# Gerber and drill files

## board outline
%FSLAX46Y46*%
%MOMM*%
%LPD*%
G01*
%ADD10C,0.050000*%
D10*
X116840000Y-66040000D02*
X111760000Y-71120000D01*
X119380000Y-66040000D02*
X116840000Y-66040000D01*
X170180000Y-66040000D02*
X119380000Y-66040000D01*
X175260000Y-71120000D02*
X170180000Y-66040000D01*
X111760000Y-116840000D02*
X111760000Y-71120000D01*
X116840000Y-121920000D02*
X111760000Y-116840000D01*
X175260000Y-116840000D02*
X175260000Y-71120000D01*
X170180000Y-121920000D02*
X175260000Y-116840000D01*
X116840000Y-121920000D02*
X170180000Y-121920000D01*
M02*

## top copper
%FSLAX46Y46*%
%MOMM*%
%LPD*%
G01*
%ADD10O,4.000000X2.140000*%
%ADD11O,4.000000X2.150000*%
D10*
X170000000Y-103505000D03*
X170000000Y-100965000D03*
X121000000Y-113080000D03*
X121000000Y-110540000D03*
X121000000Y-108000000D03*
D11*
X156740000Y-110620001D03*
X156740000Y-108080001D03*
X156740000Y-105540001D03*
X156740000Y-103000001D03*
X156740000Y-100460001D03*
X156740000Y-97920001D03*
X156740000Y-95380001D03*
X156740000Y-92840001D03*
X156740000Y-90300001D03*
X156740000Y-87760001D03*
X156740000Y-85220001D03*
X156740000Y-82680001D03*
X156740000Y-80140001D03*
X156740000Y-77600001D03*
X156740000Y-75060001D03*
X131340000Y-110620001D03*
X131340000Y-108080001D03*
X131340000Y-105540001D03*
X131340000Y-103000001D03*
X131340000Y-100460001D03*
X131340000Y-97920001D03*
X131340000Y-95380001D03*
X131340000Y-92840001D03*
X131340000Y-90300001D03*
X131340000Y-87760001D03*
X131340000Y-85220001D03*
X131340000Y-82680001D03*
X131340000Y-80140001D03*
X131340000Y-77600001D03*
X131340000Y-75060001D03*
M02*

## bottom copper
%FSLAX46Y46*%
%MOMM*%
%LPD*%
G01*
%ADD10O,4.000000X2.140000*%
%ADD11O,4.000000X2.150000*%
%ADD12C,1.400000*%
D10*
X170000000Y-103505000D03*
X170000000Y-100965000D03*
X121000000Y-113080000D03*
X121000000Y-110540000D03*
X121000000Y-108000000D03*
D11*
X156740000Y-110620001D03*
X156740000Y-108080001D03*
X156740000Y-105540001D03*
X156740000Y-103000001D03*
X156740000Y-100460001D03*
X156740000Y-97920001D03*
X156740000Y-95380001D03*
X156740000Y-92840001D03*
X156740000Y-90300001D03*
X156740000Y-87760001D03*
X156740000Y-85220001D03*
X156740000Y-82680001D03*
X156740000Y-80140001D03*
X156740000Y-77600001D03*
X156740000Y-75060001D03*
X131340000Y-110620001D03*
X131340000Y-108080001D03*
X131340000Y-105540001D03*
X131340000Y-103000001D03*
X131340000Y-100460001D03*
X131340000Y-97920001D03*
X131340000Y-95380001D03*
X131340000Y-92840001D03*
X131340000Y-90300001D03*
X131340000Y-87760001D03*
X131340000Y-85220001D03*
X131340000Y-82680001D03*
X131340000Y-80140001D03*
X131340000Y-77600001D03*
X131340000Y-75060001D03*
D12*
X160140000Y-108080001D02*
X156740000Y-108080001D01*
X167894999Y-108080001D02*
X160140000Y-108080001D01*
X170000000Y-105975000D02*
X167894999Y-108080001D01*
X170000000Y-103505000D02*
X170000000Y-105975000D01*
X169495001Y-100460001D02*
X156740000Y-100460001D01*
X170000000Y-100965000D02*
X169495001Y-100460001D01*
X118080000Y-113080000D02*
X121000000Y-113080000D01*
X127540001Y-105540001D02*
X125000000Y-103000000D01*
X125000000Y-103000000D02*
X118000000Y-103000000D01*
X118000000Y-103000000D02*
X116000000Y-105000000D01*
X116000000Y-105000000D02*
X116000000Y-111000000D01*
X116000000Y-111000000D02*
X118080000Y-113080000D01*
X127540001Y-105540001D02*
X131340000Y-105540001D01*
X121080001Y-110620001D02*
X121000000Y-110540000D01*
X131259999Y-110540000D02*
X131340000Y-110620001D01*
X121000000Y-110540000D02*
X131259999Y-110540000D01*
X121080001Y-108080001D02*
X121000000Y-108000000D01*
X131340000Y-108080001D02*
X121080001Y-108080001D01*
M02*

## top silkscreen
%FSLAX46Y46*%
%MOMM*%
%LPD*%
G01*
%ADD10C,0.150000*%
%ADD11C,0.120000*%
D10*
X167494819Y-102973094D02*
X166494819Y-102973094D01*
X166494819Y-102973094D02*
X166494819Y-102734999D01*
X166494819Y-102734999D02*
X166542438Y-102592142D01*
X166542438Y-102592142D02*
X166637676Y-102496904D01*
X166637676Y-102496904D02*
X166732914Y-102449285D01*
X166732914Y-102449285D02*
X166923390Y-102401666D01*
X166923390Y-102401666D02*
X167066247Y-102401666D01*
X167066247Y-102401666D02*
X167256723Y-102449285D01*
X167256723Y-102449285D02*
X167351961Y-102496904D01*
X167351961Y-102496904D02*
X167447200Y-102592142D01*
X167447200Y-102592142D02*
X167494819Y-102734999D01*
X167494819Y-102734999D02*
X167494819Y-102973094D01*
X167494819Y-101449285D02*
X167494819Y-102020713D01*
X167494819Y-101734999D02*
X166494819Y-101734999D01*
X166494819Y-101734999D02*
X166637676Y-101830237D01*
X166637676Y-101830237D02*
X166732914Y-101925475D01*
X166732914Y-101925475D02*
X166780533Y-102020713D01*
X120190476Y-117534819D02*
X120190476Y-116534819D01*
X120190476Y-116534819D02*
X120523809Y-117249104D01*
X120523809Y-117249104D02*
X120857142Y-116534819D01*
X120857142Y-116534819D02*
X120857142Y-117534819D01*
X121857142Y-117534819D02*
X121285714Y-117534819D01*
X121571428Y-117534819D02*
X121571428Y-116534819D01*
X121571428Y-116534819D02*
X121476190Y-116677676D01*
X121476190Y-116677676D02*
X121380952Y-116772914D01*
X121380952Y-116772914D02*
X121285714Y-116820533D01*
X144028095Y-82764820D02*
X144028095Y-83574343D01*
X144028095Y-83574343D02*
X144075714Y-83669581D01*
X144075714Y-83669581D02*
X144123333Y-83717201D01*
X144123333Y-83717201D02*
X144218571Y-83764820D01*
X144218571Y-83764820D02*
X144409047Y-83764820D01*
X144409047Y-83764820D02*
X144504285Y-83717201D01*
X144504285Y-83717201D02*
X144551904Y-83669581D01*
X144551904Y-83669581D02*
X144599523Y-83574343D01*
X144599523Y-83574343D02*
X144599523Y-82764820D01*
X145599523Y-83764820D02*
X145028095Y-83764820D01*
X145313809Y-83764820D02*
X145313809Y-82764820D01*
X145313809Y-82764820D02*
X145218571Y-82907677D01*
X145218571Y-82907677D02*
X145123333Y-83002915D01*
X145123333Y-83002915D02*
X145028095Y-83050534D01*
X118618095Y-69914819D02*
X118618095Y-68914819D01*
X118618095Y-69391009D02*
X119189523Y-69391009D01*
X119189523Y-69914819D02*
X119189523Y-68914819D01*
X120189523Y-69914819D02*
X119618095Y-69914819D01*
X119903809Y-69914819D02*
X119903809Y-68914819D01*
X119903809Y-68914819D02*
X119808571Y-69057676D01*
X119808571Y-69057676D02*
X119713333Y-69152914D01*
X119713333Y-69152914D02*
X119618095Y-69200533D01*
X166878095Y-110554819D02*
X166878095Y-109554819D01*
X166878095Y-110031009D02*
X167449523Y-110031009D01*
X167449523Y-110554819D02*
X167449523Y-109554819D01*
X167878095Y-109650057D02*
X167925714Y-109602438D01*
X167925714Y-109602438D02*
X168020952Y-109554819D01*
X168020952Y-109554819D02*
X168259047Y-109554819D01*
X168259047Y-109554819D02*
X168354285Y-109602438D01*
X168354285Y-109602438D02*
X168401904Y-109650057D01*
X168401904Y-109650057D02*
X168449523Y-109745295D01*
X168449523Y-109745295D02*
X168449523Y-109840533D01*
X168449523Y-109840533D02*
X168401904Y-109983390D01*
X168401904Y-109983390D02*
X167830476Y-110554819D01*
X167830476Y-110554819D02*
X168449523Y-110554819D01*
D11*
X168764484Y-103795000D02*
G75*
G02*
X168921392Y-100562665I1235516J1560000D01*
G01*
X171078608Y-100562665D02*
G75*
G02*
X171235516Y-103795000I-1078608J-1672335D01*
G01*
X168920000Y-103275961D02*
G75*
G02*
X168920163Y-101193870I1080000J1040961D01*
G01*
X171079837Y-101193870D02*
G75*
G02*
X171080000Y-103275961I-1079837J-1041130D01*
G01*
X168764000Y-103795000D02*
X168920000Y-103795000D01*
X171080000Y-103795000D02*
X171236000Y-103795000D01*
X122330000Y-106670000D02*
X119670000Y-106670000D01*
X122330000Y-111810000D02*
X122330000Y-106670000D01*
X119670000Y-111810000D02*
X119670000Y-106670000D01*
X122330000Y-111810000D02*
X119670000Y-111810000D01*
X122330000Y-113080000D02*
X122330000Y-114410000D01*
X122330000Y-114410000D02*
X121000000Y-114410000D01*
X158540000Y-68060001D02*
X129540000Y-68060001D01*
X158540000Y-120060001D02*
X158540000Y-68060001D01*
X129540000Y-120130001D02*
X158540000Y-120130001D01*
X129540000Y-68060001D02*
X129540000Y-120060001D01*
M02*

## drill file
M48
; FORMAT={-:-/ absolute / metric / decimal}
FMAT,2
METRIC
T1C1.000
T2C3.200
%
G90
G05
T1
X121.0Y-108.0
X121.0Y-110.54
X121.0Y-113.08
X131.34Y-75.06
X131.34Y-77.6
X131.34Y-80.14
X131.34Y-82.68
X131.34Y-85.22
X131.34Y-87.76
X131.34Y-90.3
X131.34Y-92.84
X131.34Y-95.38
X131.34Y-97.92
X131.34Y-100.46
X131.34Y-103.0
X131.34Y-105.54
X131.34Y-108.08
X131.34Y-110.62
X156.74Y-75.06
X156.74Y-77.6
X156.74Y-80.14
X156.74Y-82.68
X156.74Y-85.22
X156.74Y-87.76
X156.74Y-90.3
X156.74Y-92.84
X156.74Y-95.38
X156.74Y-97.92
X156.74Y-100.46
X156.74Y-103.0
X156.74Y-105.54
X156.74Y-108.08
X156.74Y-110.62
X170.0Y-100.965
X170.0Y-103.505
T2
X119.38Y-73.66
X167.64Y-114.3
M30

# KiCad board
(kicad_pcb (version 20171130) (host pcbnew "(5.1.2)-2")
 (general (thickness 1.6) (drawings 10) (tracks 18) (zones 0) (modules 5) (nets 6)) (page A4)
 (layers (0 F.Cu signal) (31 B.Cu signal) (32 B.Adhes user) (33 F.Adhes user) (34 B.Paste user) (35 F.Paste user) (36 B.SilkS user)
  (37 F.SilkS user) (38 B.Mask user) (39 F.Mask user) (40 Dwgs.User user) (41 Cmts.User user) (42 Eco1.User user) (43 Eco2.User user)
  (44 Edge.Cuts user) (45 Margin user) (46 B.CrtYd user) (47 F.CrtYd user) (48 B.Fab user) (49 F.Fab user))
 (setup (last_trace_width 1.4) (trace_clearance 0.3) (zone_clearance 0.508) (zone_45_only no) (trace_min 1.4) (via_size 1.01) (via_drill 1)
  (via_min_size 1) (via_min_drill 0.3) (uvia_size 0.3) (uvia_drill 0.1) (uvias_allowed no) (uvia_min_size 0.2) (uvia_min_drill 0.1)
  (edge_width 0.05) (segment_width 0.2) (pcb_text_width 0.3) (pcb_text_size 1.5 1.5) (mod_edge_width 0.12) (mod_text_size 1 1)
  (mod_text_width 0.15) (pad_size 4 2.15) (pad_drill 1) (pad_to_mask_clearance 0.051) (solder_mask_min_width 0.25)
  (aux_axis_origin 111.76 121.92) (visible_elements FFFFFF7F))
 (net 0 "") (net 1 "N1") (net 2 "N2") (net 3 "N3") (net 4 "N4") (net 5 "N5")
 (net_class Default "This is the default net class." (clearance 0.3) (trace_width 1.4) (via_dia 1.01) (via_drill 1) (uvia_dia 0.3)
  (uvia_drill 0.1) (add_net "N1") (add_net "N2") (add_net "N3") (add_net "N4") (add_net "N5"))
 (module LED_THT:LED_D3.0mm (layer F.Cu) (at 170 103.505 90)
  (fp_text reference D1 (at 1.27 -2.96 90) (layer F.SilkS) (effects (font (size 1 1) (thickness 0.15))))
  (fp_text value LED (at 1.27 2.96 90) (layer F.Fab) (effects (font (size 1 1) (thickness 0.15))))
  (fp_arc (start 1.27 0) (end -0.29 -1.235516) (angle 108.8) (layer F.SilkS) (width 0.12))
  (fp_arc (start 1.27 0) (end -0.29 1.235516) (angle -108.8) (layer F.SilkS) (width 0.12))
  (fp_arc (start 1.27 0) (end 0.229039 -1.08) (angle 87.9) (layer F.SilkS) (width 0.12))
  (fp_arc (start 1.27 0) (end 0.229039 1.08) (angle -87.9) (layer F.SilkS) (width 0.12))
  (fp_line (start -0.29 -1.236) (end -0.29 -1.08) (layer F.SilkS) (width 0.12))
  (fp_line (start -0.29 1.08) (end -0.29 1.236) (layer F.SilkS) (width 0.12))
  (pad 1 thru_hole oval (at 0 0 90) (size 2.14 4) (drill 1) (layers *.Cu *.Mask) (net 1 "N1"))
  (pad 2 thru_hole oval (at 2.54 0 90) (size 2.14 4) (drill 1) (layers *.Cu *.Mask) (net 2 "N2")))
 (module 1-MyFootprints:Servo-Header (layer F.Cu) (at 121 113.08 180)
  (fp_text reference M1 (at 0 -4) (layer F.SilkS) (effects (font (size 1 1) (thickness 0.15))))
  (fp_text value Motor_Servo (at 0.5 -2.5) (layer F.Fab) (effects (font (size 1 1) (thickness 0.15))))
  (fp_line (start -1.33 6.41) (end 1.33 6.41) (layer F.SilkS) (width 0.12))
  (fp_line (start -1.33 1.27) (end -1.33 6.41) (layer F.SilkS) (width 0.12))
  (fp_line (start 1.33 1.27) (end 1.33 6.41) (layer F.SilkS) (width 0.12))
  (fp_line (start -1.33 1.27) (end 1.33 1.27) (layer F.SilkS) (width 0.12))
  (fp_line (start -1.33 0) (end -1.33 -1.33) (layer F.SilkS) (width 0.12))
  (fp_line (start -1.33 -1.33) (end 0 -1.33) (layer F.SilkS) (width 0.12))
  (pad 1 thru_hole oval (at 0 0 180) (size 4 2.14) (drill 1) (layers *.Cu *.Mask) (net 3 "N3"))
  (pad 2 thru_hole oval (at 0 2.54 180) (size 4 2.14) (drill 1) (layers *.Cu *.Mask) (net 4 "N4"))
  (pad 3 thru_hole oval (at 0 5.08 180) (size 4 2.14) (drill 1) (layers *.Cu *.Mask) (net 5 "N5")))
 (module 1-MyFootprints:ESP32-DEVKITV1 (layer F.Cu) (at 129.54 68.060001)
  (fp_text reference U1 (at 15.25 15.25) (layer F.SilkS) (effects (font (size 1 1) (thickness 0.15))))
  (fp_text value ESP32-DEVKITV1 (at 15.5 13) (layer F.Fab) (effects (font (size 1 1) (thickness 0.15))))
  (fp_line (start 29 0) (end 0 0) (layer F.SilkS) (width 0.12))
  (fp_line (start 29 52) (end 29 0) (layer F.SilkS) (width 0.12))
  (fp_line (start 0 52.07) (end 29 52.07) (layer F.SilkS) (width 0.12))
  (fp_line (start 0 0) (end 0 52) (layer F.SilkS) (width 0.12))
  (pad 30 thru_hole oval (at 27.2 42.56) (size 4 2.15) (drill 1) (layers *.Cu *.Mask))
  (pad 29 thru_hole oval (at 27.2 40.02) (size 4 2.15) (drill 1) (layers *.Cu *.Mask) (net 1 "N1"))
  (pad 28 thru_hole oval (at 27.2 37.48) (size 4 2.15) (drill 1) (layers *.Cu *.Mask))
  (pad 27 thru_hole oval (at 27.2 34.94) (size 4 2.15) (drill 1) (layers *.Cu *.Mask))
  (pad 26 thru_hole oval (at 27.2 32.4) (size 4 2.15) (drill 1) (layers *.Cu *.Mask) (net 2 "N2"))
  (pad 25 thru_hole oval (at 27.2 29.86) (size 4 2.15) (drill 1) (layers *.Cu *.Mask))
  (pad 24 thru_hole oval (at 27.2 27.32) (size 4 2.15) (drill 1) (layers *.Cu *.Mask))
  (pad 23 thru_hole oval (at 27.2 24.78) (size 4 2.15) (drill 1) (layers *.Cu *.Mask))
  (pad 22 thru_hole oval (at 27.2 22.24) (size 4 2.15) (drill 1) (layers *.Cu *.Mask))
  (pad 21 thru_hole oval (at 27.2 19.7) (size 4 2.15) (drill 1) (layers *.Cu *.Mask))
  (pad 20 thru_hole oval (at 27.2 17.16) (size 4 2.15) (drill 1) (layers *.Cu *.Mask))
  (pad 19 thru_hole oval (at 27.2 14.62) (size 4 2.15) (drill 1) (layers *.Cu *.Mask))
  (pad 18 thru_hole oval (at 27.2 12.08) (size 4 2.15) (drill 1) (layers *.Cu *.Mask))
  (pad 17 thru_hole oval (at 27.2 9.54) (size 4 2.15) (drill 1) (layers *.Cu *.Mask))
  (pad 16 thru_hole oval (at 27.2 7) (size 4 2.15) (drill 1) (layers *.Cu *.Mask))
  (pad 15 thru_hole oval (at 1.8 42.56) (size 4 2.15) (drill 1) (layers *.Cu *.Mask) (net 4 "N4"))
  (pad 14 thru_hole oval (at 1.8 40.02) (size 4 2.15) (drill 1) (layers *.Cu *.Mask) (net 5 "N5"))
  (pad 13 thru_hole oval (at 1.8 37.48) (size 4 2.15) (drill 1) (layers *.Cu *.Mask) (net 3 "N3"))
  (pad 12 thru_hole oval (at 1.8 34.94) (size 4 2.15) (drill 1) (layers *.Cu *.Mask))
  (pad 11 thru_hole oval (at 1.8 32.4) (size 4 2.15) (drill 1) (layers *.Cu *.Mask))
  (pad 10 thru_hole oval (at 1.8 29.86) (size 4 2.15) (drill 1) (layers *.Cu *.Mask))
  (pad 9 thru_hole oval (at 1.8 27.32) (size 4 2.15) (drill 1) (layers *.Cu *.Mask))
  (pad 8 thru_hole oval (at 1.8 24.78) (size 4 2.15) (drill 1) (layers *.Cu *.Mask))
  (pad 7 thru_hole oval (at 1.8 22.24) (size 4 2.15) (drill 1) (layers *.Cu *.Mask))
  (pad 6 thru_hole oval (at 1.8 19.7) (size 4 2.15) (drill 1) (layers *.Cu *.Mask))
  (pad 5 thru_hole oval (at 1.8 17.16) (size 4 2.15) (drill 1) (layers *.Cu *.Mask))
  (pad 4 thru_hole oval (at 1.8 14.62) (size 4 2.15) (drill 1) (layers *.Cu *.Mask))
  (pad 3 thru_hole oval (at 1.8 12.08) (size 4 2.15) (drill 1) (layers *.Cu *.Mask))
  (pad 2 thru_hole oval (at 1.8 9.54) (size 4 2.15) (drill 1) (layers *.Cu *.Mask))
  (pad 1 thru_hole oval (at 1.8 7) (size 4 2.15) (drill 1) (layers *.Cu *.Mask)))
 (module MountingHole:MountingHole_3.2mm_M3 (layer F.Cu) (at 119.38 73.66)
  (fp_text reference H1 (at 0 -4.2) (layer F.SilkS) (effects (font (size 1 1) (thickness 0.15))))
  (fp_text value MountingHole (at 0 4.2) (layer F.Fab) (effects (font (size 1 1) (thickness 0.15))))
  (pad 1 np_thru_hole circle (at 0 0) (size 3.2 3.2) (drill 3.2) (layers *.Cu *.Mask)))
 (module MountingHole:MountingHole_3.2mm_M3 (layer F.Cu) (at 167.64 114.3)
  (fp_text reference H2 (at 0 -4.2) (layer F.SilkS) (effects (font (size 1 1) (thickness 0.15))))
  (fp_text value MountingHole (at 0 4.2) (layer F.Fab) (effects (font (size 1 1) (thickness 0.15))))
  (pad 1 np_thru_hole circle (at 0 0) (size 3.2 3.2) (drill 3.2) (layers *.Cu *.Mask)))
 (gr_line (start 116.84 66.04) (end 111.76 71.12) (layer Edge.Cuts) (width 0.05))
 (gr_line (start 119.38 66.04) (end 116.84 66.04) (layer Edge.Cuts) (width 0.05))
 (gr_line (start 170.18 66.04) (end 119.38 66.04) (layer Edge.Cuts) (width 0.05))
 (gr_line (start 175.26 71.12) (end 170.18 66.04) (layer Edge.Cuts) (width 0.05))
 (gr_line (start 111.76 116.84) (end 111.76 71.12) (layer Edge.Cuts) (width 0.05))
 (gr_line (start 116.84 121.92) (end 111.76 116.84) (layer Edge.Cuts) (width 0.05))
 (gr_line (start 175.26 116.84) (end 175.26 71.12) (layer Edge.Cuts) (width 0.05))
 (gr_line (start 170.18 121.92) (end 175.26 116.84) (layer Edge.Cuts) (width 0.05))
 (gr_line (start 116.84 121.92) (end 170.18 121.92) (layer Edge.Cuts) (width 0.05))
 (segment (start 160.14 108.080001) (end 156.74 108.080001) (width 1.4) (layer B.Cu) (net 1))
 (segment (start 167.894999 108.080001) (end 160.14 108.080001) (width 1.4) (layer B.Cu) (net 1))
 (segment (start 170 105.975) (end 167.894999 108.080001) (width 1.4) (layer B.Cu) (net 1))
 (segment (start 170 103.505) (end 170 105.975) (width 1.4) (layer B.Cu) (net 1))
 (segment (start 169.495001 100.460001) (end 156.74 100.460001) (width 1.4) (layer B.Cu) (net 2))
 (segment (start 170 100.965) (end 169.495001 100.460001) (width 1.4) (layer B.Cu) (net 2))
 (segment (start 118.08 113.08) (end 121 113.08) (width 1.4) (layer B.Cu) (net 3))
 (segment (start 127.540001 105.540001) (end 125 103) (width 1.4) (layer B.Cu) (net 3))
 (segment (start 125 103) (end 118 103) (width 1.4) (layer B.Cu) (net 3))
 (segment (start 118 103) (end 116 105) (width 1.4) (layer B.Cu) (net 3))
 (segment (start 116 105) (end 116 111) (width 1.4) (layer B.Cu) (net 3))
 (segment (start 116 111) (end 118.08 113.08) (width 1.4) (layer B.Cu) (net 3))
 (segment (start 127.540001 105.540001) (end 131.34 105.540001) (width 1.4) (layer B.Cu) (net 3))
 (segment (start 121.080001 110.620001) (end 121 110.54) (width 1.4) (layer B.Cu) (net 4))
 (segment (start 131.259999 110.54) (end 131.34 110.620001) (width 1.4) (layer B.Cu) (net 4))
 (segment (start 121 110.54) (end 131.259999 110.54) (width 1.4) (layer B.Cu) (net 4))
 (segment (start 121.080001 108.080001) (end 121 108) (width 1.4) (layer B.Cu) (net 5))
 (segment (start 131.34 108.080001) (end 121.080001 108.080001) (width 1.4) (layer B.Cu) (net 5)))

